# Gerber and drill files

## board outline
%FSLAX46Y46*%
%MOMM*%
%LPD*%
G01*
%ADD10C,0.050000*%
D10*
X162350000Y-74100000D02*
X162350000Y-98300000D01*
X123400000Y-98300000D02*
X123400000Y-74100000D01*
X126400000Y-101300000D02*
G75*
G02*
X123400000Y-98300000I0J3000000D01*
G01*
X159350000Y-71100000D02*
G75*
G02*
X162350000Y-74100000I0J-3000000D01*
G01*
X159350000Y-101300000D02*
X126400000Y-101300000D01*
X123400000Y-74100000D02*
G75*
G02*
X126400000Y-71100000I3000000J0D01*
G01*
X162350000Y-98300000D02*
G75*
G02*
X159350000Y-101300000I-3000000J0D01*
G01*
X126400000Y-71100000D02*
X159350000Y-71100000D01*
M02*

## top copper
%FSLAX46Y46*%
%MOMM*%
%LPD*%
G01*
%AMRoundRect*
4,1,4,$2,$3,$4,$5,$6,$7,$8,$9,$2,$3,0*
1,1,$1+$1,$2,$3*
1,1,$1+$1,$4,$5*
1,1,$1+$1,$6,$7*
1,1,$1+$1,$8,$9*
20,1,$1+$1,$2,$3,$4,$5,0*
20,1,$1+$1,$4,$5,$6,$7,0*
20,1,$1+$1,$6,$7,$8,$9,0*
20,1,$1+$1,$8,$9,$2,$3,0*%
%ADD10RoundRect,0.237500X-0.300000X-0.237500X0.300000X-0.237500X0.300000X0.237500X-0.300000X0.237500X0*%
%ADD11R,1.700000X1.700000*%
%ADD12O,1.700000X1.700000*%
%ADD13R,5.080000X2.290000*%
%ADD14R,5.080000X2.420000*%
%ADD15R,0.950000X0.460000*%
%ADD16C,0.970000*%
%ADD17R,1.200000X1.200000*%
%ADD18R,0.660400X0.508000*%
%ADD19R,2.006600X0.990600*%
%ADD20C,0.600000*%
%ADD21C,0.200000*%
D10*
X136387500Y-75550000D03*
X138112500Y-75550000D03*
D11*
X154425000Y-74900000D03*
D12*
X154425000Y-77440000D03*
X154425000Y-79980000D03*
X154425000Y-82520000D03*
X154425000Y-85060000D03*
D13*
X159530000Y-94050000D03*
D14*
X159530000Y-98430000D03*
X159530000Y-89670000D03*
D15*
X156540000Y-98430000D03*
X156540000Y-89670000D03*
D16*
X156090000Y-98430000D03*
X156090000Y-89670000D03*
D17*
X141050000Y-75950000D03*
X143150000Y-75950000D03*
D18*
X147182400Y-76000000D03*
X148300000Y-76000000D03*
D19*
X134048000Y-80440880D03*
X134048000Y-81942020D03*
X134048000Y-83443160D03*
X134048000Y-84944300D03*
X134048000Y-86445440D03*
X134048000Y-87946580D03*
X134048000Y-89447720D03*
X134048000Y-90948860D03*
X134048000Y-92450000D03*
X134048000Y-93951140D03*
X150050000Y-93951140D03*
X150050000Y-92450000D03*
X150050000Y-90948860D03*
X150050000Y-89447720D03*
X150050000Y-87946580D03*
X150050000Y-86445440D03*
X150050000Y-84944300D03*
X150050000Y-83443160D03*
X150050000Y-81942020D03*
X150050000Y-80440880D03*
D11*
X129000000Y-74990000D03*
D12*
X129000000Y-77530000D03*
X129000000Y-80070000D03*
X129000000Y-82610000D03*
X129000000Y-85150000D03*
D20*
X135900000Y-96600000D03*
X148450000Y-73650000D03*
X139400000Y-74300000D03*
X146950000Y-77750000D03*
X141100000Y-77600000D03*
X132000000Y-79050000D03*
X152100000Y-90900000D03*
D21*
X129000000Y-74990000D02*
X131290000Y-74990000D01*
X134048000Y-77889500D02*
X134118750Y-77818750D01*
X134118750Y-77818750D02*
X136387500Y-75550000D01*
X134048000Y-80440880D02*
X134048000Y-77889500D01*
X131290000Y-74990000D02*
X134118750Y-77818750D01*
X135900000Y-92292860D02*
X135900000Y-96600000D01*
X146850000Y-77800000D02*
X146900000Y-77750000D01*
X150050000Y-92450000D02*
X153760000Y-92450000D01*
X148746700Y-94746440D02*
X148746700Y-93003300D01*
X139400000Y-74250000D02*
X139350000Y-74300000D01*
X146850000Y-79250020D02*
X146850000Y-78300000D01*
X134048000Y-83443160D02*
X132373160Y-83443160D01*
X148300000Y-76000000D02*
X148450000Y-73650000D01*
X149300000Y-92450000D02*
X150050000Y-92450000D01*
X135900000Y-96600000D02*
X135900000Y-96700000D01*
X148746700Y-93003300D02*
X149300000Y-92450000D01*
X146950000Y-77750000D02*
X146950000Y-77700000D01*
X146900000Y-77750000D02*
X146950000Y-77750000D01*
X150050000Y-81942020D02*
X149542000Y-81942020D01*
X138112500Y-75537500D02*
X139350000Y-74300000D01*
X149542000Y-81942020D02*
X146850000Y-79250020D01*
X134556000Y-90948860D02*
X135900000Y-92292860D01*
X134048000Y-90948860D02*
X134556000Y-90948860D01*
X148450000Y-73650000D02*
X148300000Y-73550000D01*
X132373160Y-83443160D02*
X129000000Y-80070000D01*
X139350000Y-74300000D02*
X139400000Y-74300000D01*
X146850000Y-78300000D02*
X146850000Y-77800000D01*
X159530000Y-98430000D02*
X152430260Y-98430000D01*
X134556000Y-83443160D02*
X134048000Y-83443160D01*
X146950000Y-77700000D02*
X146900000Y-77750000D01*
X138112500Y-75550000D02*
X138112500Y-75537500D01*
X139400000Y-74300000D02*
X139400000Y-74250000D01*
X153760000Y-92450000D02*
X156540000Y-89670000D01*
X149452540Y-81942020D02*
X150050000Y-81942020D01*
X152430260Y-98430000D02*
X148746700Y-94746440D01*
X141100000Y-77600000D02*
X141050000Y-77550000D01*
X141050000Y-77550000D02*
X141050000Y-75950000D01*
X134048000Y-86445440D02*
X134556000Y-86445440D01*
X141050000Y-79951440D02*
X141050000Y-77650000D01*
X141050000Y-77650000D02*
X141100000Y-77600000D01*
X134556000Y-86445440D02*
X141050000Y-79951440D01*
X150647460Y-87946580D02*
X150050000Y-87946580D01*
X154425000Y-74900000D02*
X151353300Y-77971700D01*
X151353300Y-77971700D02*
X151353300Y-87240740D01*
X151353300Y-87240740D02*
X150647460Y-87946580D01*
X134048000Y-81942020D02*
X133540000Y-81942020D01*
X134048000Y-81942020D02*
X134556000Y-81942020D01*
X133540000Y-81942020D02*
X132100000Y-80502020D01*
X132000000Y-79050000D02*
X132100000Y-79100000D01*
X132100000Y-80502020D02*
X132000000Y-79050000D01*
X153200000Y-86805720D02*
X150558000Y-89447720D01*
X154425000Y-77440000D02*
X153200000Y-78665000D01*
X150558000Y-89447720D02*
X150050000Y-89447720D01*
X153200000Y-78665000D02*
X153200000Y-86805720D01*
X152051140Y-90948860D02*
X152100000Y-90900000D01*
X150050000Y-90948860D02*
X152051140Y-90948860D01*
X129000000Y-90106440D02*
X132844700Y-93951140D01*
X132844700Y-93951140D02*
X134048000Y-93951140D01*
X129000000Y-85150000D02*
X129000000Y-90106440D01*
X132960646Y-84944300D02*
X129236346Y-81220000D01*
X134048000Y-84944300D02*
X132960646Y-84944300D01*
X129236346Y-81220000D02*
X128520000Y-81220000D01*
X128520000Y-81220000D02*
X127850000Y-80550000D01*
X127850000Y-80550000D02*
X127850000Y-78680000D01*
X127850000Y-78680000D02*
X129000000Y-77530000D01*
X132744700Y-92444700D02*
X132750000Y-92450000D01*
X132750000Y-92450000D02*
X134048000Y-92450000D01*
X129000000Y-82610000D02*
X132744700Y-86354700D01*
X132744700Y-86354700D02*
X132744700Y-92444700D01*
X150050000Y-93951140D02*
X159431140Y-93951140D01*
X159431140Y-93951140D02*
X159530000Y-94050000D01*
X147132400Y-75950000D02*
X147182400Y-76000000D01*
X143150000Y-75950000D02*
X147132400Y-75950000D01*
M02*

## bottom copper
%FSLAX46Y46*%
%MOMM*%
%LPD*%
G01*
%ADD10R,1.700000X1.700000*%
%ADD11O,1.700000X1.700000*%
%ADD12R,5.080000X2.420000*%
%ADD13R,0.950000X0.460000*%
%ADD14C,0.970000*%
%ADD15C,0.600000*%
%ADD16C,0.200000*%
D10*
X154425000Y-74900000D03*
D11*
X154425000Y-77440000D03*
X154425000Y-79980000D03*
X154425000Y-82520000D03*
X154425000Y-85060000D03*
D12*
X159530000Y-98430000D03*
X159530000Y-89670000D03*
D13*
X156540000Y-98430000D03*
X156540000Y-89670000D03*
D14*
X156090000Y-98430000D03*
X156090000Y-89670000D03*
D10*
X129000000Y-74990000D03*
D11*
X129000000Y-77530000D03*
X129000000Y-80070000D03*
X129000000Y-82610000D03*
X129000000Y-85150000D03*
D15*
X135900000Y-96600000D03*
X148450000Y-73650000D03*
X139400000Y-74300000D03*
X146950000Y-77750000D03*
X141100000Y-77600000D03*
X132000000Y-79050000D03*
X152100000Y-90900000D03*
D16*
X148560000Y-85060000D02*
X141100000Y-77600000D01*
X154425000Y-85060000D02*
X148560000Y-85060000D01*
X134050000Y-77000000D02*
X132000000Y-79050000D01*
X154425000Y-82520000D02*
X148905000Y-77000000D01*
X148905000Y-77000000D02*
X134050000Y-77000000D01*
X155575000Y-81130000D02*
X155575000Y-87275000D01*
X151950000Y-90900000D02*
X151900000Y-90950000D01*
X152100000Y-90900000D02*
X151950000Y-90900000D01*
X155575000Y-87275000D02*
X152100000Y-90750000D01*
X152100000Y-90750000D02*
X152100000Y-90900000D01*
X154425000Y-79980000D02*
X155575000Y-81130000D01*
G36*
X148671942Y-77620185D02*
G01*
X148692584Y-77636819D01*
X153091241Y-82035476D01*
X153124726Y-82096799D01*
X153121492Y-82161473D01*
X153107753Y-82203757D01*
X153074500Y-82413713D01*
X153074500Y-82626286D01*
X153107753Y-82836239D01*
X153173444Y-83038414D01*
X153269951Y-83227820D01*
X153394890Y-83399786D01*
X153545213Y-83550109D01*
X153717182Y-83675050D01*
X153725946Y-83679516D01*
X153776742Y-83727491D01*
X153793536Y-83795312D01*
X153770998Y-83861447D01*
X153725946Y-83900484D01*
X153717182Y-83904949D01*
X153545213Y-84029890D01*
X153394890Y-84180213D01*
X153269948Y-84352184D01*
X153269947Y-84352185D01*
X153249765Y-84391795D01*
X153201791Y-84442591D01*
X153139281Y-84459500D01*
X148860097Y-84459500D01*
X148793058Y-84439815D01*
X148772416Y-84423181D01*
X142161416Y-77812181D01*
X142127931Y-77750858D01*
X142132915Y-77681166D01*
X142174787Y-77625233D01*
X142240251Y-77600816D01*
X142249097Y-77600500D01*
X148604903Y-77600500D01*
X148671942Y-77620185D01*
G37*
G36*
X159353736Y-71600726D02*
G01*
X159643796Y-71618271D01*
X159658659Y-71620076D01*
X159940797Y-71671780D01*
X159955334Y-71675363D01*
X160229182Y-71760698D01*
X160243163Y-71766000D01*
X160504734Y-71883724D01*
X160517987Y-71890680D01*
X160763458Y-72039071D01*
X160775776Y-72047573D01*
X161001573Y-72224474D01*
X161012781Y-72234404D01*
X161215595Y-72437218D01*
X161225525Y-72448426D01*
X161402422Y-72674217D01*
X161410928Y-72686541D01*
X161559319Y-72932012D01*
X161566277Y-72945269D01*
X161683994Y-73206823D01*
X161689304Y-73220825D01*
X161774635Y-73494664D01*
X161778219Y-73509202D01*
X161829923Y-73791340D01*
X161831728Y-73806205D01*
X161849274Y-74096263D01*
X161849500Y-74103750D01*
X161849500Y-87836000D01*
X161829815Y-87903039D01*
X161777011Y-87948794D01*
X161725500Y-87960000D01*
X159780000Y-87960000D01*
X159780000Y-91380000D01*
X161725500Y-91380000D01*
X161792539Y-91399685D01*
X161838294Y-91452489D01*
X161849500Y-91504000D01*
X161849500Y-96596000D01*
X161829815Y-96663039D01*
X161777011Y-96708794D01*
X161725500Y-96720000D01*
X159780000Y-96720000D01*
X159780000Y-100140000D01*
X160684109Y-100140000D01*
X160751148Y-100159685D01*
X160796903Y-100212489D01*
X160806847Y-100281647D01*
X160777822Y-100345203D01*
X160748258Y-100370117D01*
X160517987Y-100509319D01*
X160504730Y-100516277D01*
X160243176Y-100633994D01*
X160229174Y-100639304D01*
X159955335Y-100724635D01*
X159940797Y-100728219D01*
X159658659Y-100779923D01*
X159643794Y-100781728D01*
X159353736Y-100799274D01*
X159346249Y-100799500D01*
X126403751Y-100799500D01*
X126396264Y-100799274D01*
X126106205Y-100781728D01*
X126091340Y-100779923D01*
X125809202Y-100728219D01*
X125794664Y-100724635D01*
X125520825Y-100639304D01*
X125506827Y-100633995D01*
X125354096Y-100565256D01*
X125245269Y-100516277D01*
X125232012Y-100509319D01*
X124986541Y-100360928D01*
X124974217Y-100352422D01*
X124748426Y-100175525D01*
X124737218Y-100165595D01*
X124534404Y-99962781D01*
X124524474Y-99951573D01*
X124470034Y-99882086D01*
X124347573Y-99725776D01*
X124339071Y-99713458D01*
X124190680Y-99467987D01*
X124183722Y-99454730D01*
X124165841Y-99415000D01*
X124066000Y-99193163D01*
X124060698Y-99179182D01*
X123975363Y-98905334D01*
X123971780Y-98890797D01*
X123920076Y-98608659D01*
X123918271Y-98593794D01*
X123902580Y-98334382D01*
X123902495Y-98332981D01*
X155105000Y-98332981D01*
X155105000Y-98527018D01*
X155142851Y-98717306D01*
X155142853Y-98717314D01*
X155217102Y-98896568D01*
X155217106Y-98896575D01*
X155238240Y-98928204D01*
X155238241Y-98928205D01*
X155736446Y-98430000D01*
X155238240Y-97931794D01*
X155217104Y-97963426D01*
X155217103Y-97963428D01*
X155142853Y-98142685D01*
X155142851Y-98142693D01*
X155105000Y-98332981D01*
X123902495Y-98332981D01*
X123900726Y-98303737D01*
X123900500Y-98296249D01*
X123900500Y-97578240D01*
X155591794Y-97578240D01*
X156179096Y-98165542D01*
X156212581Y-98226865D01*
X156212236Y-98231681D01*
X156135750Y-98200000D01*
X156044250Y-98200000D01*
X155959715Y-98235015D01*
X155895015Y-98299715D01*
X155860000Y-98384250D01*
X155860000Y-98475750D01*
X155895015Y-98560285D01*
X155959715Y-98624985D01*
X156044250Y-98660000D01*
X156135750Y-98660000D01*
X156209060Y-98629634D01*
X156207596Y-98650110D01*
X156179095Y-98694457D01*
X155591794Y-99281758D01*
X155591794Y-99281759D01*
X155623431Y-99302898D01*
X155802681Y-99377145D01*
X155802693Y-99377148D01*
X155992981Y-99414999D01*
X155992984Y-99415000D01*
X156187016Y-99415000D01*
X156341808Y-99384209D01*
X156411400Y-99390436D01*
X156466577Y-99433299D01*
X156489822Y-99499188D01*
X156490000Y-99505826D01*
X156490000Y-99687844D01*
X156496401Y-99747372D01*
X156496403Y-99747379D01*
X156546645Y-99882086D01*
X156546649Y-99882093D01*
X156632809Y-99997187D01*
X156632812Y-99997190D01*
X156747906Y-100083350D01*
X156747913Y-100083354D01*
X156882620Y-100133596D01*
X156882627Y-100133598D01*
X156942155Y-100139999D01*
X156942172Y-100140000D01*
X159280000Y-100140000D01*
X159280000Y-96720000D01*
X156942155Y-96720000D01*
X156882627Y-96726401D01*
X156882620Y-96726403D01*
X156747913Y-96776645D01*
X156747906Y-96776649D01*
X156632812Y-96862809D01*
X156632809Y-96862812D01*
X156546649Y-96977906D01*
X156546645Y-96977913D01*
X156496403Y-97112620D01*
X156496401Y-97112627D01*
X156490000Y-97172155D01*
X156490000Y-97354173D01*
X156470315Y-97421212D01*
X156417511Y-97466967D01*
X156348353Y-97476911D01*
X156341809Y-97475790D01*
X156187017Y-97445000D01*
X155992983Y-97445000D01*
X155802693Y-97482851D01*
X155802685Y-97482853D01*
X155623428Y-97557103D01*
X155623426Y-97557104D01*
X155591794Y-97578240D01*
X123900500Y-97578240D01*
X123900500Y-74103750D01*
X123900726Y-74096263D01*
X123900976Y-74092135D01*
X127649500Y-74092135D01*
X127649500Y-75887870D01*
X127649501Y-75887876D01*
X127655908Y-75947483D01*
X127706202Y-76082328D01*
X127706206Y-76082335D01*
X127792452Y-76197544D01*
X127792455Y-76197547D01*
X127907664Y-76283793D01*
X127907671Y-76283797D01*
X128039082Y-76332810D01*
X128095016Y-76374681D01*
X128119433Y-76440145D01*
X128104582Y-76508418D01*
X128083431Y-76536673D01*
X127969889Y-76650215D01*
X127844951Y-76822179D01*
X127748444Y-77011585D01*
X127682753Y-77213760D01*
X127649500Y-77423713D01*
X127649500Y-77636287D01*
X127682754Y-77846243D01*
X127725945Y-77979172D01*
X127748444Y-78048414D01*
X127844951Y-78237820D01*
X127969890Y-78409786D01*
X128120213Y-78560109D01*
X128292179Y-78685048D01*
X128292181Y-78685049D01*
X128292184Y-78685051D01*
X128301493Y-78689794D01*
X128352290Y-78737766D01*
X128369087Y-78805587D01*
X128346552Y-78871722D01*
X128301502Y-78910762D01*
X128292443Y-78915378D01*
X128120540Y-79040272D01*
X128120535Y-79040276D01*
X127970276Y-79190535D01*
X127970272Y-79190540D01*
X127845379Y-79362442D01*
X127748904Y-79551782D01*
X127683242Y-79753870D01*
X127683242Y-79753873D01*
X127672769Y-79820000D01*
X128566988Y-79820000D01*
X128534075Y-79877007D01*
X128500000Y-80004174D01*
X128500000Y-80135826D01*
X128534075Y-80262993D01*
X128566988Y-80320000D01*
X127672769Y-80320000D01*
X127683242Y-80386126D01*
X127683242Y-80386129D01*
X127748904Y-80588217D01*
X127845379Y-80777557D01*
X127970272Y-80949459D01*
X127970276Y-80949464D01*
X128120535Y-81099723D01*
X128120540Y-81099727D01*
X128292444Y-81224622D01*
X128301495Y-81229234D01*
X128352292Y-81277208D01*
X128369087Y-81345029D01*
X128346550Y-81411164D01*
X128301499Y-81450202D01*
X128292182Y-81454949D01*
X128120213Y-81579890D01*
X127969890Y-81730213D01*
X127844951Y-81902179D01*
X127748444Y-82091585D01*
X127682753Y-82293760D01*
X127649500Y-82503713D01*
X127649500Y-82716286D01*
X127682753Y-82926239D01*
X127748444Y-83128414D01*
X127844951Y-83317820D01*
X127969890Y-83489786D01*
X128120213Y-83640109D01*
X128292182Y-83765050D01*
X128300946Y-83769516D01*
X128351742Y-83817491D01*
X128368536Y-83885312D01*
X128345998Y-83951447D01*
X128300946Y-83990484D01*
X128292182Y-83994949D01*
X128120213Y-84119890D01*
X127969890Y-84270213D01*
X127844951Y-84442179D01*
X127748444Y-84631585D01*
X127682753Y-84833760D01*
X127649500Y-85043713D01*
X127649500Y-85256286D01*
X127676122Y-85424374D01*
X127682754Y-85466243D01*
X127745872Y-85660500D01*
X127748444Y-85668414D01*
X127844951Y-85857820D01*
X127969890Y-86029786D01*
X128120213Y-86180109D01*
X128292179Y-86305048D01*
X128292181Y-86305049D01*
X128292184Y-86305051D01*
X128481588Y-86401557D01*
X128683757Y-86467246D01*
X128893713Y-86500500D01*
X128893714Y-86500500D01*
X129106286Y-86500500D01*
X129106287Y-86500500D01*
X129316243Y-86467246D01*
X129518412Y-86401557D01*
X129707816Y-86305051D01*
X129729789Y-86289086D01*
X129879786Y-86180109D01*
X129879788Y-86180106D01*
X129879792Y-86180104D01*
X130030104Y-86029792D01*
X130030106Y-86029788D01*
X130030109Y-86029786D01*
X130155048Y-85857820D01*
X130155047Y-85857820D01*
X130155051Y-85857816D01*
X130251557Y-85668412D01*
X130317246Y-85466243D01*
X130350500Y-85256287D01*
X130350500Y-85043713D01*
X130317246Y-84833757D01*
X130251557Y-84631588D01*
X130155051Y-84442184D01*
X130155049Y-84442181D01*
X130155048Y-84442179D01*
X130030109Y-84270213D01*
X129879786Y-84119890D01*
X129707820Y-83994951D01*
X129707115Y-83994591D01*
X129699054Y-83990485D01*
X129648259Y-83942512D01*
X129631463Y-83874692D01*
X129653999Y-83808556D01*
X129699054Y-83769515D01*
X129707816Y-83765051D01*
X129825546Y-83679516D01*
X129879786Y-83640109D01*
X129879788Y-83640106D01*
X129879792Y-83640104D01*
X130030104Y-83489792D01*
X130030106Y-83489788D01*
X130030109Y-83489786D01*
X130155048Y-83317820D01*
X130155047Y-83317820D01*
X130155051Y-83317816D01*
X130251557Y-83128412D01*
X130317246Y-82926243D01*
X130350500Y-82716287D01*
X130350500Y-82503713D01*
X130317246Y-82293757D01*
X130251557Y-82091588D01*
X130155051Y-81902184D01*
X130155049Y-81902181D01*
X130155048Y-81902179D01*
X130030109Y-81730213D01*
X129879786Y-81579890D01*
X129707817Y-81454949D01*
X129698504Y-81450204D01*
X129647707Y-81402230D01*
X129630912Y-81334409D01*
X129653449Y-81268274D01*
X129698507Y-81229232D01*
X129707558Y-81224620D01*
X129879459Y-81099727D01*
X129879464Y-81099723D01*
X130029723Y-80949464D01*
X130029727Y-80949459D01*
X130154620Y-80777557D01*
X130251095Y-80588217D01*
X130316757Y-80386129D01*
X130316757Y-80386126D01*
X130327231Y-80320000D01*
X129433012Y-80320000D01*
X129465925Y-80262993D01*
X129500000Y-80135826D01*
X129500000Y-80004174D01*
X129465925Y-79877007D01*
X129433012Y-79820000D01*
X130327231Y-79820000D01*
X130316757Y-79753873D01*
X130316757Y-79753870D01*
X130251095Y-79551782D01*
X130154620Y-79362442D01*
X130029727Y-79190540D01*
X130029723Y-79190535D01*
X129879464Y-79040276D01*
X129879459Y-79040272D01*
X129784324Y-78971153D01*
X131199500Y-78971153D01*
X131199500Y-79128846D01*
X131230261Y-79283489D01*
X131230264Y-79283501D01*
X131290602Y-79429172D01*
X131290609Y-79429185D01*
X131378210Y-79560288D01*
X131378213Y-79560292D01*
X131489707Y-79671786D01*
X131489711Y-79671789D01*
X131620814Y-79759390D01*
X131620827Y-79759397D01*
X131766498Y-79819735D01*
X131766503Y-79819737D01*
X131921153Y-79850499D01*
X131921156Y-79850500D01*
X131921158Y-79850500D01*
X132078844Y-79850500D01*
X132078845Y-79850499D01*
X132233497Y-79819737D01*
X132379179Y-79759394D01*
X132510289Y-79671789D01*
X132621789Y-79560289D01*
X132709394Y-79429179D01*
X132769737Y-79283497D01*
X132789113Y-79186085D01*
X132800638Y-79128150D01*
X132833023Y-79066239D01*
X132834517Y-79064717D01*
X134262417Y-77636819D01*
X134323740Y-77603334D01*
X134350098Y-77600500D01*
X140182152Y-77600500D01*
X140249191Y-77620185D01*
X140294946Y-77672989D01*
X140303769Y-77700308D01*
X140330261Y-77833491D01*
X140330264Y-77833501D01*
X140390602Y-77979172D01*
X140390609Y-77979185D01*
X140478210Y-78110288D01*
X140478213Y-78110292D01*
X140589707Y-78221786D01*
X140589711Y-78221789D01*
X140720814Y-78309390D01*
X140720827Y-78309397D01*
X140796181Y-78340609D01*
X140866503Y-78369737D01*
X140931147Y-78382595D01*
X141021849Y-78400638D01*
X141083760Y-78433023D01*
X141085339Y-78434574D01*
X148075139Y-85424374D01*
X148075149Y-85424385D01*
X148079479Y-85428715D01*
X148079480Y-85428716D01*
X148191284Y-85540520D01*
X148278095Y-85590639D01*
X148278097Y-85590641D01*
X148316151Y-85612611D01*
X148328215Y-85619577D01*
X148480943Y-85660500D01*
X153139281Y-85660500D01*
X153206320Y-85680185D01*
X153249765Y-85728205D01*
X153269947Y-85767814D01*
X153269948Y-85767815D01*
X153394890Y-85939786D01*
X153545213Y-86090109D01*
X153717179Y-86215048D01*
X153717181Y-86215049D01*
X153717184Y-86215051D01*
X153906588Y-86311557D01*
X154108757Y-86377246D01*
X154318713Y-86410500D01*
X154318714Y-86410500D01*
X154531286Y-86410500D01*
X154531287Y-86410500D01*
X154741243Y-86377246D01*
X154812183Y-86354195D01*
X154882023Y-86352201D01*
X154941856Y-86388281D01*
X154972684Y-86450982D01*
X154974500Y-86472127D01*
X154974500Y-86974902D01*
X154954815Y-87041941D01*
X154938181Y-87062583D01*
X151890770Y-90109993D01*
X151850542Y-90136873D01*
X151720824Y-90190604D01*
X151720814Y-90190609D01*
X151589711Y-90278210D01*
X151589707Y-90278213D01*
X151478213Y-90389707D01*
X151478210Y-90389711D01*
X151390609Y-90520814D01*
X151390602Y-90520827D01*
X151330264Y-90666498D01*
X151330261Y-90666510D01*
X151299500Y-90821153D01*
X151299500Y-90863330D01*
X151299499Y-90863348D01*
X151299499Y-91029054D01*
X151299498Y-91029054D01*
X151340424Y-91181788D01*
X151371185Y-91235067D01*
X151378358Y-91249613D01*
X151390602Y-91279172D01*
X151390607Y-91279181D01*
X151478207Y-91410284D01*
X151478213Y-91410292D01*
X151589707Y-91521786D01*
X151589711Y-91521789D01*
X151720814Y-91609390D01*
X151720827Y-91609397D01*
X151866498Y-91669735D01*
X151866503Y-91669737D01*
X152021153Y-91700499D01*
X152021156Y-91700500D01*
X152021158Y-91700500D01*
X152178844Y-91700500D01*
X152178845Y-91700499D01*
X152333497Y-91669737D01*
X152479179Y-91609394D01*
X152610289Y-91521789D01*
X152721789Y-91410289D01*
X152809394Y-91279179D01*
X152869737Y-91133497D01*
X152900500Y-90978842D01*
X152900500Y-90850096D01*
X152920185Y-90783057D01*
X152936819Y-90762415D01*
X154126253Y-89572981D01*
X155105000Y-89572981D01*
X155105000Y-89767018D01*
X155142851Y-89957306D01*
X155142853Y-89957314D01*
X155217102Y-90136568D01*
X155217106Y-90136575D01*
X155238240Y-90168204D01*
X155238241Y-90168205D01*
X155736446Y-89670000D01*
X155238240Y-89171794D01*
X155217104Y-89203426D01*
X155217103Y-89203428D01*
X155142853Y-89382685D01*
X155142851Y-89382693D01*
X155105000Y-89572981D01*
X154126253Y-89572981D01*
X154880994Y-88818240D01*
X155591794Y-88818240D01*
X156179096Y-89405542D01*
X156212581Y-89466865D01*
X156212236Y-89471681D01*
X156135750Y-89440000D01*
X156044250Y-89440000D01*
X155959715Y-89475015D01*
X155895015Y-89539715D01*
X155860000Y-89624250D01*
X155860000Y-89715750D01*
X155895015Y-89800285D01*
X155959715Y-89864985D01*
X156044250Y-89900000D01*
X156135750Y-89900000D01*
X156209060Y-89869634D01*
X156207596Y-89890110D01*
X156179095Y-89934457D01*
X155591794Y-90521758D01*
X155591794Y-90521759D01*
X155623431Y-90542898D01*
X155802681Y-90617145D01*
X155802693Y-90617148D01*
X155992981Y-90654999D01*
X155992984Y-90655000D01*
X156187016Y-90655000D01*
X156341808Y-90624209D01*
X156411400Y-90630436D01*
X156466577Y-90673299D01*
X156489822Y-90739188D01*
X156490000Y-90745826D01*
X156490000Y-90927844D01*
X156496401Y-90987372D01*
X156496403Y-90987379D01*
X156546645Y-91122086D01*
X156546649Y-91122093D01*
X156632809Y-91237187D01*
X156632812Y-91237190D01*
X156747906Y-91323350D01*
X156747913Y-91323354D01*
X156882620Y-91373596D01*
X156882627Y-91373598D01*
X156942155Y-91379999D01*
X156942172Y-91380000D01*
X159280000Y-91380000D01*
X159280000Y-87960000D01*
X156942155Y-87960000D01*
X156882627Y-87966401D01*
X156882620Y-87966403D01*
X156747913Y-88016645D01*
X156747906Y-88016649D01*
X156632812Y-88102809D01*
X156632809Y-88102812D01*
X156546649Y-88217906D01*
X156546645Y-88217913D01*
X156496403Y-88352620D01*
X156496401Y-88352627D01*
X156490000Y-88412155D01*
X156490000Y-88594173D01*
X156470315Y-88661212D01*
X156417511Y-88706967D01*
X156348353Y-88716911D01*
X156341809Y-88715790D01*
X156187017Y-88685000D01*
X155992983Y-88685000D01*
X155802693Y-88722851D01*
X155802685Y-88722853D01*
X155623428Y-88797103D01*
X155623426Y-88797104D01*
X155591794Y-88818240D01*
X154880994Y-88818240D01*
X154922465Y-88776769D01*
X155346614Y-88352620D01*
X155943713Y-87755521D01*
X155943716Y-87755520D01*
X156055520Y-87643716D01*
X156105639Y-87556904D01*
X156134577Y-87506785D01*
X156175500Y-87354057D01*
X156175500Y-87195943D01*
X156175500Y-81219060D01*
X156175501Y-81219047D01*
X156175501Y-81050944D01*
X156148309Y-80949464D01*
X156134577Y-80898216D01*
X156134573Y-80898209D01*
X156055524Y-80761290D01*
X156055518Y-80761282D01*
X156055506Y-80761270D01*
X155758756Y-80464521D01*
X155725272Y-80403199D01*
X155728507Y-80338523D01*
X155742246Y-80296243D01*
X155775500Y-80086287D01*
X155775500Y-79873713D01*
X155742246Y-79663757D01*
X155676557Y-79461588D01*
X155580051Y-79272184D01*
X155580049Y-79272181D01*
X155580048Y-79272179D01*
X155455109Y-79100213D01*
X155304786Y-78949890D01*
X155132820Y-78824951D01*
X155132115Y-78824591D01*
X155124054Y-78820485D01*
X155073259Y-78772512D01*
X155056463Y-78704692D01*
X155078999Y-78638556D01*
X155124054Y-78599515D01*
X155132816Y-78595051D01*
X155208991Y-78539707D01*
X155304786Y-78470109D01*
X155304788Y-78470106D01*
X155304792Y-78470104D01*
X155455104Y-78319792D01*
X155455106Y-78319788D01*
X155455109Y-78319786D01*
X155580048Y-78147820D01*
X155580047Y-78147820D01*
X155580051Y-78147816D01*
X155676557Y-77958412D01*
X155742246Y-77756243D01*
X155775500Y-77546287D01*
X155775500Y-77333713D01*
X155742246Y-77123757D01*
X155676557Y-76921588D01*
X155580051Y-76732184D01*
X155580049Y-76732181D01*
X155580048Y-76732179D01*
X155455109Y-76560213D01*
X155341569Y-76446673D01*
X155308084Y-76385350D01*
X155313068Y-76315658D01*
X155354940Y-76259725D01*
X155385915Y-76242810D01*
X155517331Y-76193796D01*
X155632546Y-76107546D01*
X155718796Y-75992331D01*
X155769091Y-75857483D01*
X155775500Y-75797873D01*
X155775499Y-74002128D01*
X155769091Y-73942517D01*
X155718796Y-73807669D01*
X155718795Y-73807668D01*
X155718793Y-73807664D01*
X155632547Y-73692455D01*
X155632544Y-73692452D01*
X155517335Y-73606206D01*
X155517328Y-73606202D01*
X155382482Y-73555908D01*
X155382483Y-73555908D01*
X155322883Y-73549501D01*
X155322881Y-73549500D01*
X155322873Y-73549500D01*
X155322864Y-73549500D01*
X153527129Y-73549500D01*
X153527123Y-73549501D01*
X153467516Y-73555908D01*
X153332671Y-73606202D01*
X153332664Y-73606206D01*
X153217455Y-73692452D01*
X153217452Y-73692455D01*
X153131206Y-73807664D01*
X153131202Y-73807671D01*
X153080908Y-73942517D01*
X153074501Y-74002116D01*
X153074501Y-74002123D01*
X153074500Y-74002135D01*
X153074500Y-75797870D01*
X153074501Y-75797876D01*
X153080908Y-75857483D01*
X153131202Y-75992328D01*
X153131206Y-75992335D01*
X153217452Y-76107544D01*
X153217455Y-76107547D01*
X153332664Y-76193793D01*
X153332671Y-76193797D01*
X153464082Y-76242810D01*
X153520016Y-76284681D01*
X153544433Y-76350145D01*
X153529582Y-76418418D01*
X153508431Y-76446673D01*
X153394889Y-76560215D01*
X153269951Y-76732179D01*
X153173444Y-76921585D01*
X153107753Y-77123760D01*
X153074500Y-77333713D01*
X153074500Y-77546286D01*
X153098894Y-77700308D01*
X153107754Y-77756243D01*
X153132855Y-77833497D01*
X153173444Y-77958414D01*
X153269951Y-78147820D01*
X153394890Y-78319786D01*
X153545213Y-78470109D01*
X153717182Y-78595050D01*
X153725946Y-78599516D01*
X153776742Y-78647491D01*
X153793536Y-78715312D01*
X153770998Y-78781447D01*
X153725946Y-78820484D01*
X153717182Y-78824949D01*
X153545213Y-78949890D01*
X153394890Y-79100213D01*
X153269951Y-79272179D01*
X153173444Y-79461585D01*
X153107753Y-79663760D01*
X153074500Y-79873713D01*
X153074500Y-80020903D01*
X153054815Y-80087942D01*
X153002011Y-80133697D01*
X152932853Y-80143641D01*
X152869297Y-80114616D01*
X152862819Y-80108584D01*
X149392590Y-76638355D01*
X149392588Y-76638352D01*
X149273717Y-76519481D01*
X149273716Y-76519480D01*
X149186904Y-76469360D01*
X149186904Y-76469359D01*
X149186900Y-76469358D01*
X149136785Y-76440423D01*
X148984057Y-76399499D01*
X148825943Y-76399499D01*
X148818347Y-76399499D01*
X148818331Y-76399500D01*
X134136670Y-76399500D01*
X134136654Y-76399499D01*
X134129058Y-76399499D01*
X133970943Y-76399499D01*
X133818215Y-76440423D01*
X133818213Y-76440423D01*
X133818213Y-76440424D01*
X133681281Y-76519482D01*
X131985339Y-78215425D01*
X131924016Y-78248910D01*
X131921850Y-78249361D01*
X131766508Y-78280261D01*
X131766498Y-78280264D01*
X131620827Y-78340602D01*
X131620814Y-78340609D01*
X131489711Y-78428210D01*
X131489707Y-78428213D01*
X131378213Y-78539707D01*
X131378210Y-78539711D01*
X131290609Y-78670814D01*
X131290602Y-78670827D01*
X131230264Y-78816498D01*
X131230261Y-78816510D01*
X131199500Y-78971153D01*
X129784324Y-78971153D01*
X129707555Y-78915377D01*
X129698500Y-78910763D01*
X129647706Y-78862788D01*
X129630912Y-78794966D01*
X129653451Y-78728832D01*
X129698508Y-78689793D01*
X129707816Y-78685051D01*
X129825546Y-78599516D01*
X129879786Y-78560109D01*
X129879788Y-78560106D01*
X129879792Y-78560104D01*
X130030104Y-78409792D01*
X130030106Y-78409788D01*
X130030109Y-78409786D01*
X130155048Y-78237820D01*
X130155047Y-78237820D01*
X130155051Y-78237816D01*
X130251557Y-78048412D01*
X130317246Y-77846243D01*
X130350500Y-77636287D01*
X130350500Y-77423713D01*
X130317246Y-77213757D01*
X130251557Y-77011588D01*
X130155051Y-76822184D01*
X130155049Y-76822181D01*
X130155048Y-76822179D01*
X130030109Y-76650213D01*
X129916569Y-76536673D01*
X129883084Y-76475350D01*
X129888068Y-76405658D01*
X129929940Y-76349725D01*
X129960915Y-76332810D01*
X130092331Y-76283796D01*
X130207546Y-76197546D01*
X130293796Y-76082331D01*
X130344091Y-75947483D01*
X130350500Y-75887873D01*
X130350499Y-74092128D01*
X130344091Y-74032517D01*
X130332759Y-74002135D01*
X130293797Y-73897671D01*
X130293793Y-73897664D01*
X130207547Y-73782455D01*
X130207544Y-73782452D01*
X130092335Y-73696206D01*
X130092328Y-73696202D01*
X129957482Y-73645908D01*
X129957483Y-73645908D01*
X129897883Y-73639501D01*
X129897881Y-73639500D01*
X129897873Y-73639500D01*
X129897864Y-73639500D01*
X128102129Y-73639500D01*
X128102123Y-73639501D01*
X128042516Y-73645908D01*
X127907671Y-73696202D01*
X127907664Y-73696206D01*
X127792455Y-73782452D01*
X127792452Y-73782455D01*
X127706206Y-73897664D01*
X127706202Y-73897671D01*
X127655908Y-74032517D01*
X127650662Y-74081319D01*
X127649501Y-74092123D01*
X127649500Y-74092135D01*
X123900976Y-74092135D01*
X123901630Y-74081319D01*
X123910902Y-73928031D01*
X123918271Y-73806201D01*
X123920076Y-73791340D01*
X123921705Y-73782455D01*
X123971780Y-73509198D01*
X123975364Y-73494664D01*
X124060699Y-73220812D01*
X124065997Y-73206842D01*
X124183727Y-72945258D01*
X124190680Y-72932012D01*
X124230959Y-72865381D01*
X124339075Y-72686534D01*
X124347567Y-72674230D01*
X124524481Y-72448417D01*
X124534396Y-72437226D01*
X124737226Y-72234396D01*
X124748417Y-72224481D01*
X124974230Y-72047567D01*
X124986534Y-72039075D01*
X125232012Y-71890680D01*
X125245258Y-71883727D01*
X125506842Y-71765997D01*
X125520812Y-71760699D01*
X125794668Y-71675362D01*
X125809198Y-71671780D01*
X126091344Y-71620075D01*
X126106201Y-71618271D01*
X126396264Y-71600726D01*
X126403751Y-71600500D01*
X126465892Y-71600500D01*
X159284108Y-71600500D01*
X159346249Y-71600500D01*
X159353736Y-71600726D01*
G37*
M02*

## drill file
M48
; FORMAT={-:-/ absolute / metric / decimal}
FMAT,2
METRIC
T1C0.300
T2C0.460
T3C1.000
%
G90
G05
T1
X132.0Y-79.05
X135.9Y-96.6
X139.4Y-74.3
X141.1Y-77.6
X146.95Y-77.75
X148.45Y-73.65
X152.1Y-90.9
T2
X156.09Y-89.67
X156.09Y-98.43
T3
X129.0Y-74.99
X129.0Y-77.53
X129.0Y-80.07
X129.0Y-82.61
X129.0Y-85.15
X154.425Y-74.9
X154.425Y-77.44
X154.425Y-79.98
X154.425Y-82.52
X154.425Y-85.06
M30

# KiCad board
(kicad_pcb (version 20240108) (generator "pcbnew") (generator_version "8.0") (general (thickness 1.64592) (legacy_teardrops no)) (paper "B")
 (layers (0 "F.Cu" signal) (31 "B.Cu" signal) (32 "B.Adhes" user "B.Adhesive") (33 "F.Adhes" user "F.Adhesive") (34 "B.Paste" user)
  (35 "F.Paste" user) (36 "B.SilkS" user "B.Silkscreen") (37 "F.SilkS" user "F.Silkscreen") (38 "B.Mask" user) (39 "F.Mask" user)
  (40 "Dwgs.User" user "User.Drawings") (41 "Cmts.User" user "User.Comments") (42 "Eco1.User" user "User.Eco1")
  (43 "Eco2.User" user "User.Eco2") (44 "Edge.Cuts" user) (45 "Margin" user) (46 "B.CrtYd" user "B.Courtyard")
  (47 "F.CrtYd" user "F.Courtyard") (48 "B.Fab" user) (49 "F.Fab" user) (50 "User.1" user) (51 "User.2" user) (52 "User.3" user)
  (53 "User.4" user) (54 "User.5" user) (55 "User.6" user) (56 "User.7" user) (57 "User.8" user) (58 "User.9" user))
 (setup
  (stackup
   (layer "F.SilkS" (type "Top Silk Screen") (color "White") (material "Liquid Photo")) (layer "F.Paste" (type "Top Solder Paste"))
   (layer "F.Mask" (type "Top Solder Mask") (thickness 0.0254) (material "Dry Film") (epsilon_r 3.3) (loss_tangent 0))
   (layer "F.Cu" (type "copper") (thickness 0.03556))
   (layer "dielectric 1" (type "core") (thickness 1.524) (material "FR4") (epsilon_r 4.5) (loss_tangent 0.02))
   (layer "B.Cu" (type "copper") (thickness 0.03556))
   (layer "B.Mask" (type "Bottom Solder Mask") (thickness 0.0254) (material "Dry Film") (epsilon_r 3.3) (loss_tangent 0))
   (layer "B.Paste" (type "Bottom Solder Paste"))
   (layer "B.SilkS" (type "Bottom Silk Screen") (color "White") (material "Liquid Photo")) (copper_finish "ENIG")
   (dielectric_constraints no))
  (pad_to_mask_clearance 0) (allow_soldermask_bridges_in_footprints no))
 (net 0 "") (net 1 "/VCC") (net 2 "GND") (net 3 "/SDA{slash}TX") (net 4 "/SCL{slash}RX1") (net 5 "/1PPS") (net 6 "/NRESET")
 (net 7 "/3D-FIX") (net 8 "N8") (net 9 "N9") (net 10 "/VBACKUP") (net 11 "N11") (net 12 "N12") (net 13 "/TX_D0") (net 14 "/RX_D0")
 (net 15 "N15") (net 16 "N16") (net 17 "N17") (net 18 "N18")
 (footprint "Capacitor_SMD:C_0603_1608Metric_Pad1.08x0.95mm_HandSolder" (layer "F.Cu") (at 137.25 75.55)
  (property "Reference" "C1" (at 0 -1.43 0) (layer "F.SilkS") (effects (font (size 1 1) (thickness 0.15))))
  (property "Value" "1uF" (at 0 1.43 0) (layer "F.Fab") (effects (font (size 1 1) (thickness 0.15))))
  (pad "1" smd roundrect (at -0.8625 0) (size 1.075 0.95) (layers "F.Cu" "F.Paste" "F.Mask") (roundrect_rratio 0.25) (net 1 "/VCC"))
  (pad "2" smd roundrect (at 0.8625 0) (size 1.075 0.95) (layers "F.Cu" "F.Paste" "F.Mask") (roundrect_rratio 0.25) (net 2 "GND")))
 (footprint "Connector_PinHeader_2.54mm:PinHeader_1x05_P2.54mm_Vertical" (layer "F.Cu") (at 154.425 74.9)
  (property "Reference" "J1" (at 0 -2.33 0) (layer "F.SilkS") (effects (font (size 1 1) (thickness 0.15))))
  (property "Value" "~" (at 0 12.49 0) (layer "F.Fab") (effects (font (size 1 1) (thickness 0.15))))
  (pad "1" thru_hole rect (at 0 0) (size 1.7 1.7) (drill 1) (layers "*.Cu" "*.Mask") (remove_unused_layers no) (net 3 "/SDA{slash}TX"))
  (pad "2" thru_hole oval (at 0 2.54) (size 1.7 1.7) (drill 1) (layers "*.Cu" "*.Mask") (remove_unused_layers no) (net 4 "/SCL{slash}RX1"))
  (pad "3" thru_hole oval (at 0 5.08) (size 1.7 1.7) (drill 1) (layers "*.Cu" "*.Mask") (remove_unused_layers no) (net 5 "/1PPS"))
  (pad "4" thru_hole oval (at 0 7.62) (size 1.7 1.7) (drill 1) (layers "*.Cu" "*.Mask") (remove_unused_layers no) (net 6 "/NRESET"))
  (pad "5" thru_hole oval (at 0 10.16) (size 1.7 1.7) (drill 1) (layers "*.Cu" "*.Mask") (remove_unused_layers no) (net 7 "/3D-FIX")))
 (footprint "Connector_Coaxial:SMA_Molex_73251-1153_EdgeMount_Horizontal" (layer "F.Cu") (at 157.81 94.05 180)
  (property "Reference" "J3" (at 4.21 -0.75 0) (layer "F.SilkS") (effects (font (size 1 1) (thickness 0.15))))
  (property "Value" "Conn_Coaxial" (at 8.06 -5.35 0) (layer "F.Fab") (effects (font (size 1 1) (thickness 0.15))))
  (pad "1" smd rect (at -1.72 0 180) (size 5.08 2.29) (layers "F.Cu" "F.Paste" "F.Mask") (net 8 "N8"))
  (pad "2" smd rect (at -1.72 -4.38 180) (size 5.08 2.42) (layers "F.Cu" "F.Paste" "F.Mask") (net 2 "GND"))
  (pad "2" smd rect (at -1.72 -4.38 180) (size 5.08 2.42) (layers "B.Cu" "B.Paste" "B.Mask") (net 2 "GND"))
  (pad "2" smd rect (at -1.72 4.38 180) (size 5.08 2.42) (layers "F.Cu" "F.Paste" "F.Mask") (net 2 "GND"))
  (pad "2" smd rect (at -1.72 4.38 180) (size 5.08 2.42) (layers "B.Cu" "B.Paste" "B.Mask") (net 2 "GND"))
  (pad "2" smd rect (at 1.27 -4.38 180) (size 0.95 0.46) (layers "F.Cu") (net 2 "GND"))
  (pad "2" smd rect (at 1.27 -4.38 180) (size 0.95 0.46) (layers "B.Cu") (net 2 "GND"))
  (pad "2" smd rect (at 1.27 4.38 180) (size 0.95 0.46) (layers "F.Cu") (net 2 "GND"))
  (pad "2" smd rect (at 1.27 4.38 180) (size 0.95 0.46) (layers "B.Cu") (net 2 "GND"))
  (pad "2" thru_hole circle (at 1.72 -4.38 180) (size 0.97 0.97) (drill 0.46) (layers "*.Cu") (remove_unused_layers no) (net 2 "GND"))
  (pad "2" thru_hole circle (at 1.72 4.38 180) (size 0.97 0.97) (drill 0.46) (layers "*.Cu") (remove_unused_layers no) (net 2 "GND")))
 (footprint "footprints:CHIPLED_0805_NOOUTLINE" (layer "F.Cu") (at 142.1 75.95 -90)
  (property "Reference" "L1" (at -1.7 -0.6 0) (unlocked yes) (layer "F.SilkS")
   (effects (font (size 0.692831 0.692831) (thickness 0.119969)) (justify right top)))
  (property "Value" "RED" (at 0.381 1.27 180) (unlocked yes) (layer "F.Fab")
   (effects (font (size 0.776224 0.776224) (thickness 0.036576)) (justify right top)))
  (pad "A" smd rect (at 0 1.05 270) (size 1.2 1.2) (layers "F.Cu" "F.Paste" "F.Mask") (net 7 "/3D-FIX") (solder_mask_margin 0.0508)
   (thermal_bridge_angle 0))
  (pad "C" smd rect (at 0 -1.05 270) (size 1.2 1.2) (layers "F.Cu" "F.Paste" "F.Mask") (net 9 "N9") (solder_mask_margin 0.0508)
   (thermal_bridge_angle 0)))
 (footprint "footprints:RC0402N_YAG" (layer "F.Cu") (at 147.7412 76)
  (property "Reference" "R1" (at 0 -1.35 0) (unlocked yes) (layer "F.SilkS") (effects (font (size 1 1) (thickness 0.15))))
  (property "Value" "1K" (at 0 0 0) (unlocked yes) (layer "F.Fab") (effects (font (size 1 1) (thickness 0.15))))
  (pad "1" smd rect (at -0.5588 0) (size 0.6604 0.508) (layers "F.Cu" "F.Paste" "F.Mask") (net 9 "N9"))
  (pad "2" smd rect (at 0.5588 0) (size 0.6604 0.508) (layers "F.Cu" "F.Paste" "F.Mask") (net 2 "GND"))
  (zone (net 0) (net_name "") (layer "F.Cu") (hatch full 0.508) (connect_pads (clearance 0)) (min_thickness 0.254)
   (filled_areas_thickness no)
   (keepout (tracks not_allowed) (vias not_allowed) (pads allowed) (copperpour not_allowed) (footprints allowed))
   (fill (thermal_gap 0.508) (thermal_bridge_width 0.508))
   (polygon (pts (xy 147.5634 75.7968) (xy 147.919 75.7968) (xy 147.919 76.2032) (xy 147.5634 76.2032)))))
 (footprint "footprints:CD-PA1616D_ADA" (layer "F.Cu") (at 142.049 87.19601)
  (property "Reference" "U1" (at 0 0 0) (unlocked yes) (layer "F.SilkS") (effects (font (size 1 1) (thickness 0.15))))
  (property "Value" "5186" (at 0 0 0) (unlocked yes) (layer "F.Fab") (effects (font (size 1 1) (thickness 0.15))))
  (pad "1" smd rect (at -8.001 -6.75513) (size 2.0066 0.9906) (layers "F.Cu" "F.Paste" "F.Mask") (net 1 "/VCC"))
  (pad "2" smd rect (at -8.001 -5.25399) (size 2.0066 0.9906) (layers "F.Cu" "F.Paste" "F.Mask") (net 6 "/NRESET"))
  (pad "3" smd rect (at -8.001 -3.75285) (size 2.0066 0.9906) (layers "F.Cu" "F.Paste" "F.Mask") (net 2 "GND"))
  (pad "4" smd rect (at -8.001 -2.25171) (size 2.0066 0.9906) (layers "F.Cu" "F.Paste" "F.Mask") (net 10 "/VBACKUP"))
  (pad "5" smd rect (at -8.001 -0.75057) (size 2.0066 0.9906) (layers "F.Cu" "F.Paste" "F.Mask") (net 7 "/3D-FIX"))
  (pad "6" smd rect (at -8.001 0.75057) (size 2.0066 0.9906) (layers "F.Cu" "F.Paste" "F.Mask") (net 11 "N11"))
  (pad "7" smd rect (at -8.001 2.25171) (size 2.0066 0.9906) (layers "F.Cu" "F.Paste" "F.Mask") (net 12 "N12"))
  (pad "8" smd rect (at -8.001 3.75285) (size 2.0066 0.9906) (layers "F.Cu" "F.Paste" "F.Mask") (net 2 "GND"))
  (pad "9" smd rect (at -8.001 5.25399) (size 2.0066 0.9906) (layers "F.Cu" "F.Paste" "F.Mask") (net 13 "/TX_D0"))
  (pad "10" smd rect (at -8.001 6.75513) (size 2.0066 0.9906) (layers "F.Cu" "F.Paste" "F.Mask") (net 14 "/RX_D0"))
  (pad "11" smd rect (at 8.001 6.75513) (size 2.0066 0.9906) (layers "F.Cu" "F.Paste" "F.Mask") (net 8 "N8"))
  (pad "12" smd rect (at 8.001 5.25399) (size 2.0066 0.9906) (layers "F.Cu" "F.Paste" "F.Mask") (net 2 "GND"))
  (pad "13" smd rect (at 8.001 3.75285) (size 2.0066 0.9906) (layers "F.Cu" "F.Paste" "F.Mask") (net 5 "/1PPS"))
  (pad "14" smd rect (at 8.001 2.25171) (size 2.0066 0.9906) (layers "F.Cu" "F.Paste" "F.Mask") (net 4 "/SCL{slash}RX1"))
  (pad "15" smd rect (at 8.001 0.75057) (size 2.0066 0.9906) (layers "F.Cu" "F.Paste" "F.Mask") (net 3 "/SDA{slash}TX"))
  (pad "16" smd rect (at 8.001 -0.75057) (size 2.0066 0.9906) (layers "F.Cu" "F.Paste" "F.Mask") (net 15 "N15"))
  (pad "17" smd rect (at 8.001 -2.25171) (size 2.0066 0.9906) (layers "F.Cu" "F.Paste" "F.Mask") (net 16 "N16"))
  (pad "18" smd rect (at 8.001 -3.75285) (size 2.0066 0.9906) (layers "F.Cu" "F.Paste" "F.Mask") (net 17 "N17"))
  (pad "19" smd rect (at 8.001 -5.25399) (size 2.0066 0.9906) (layers "F.Cu" "F.Paste" "F.Mask") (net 2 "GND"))
  (pad "20" smd rect (at 8.001 -6.75513) (size 2.0066 0.9906) (layers "F.Cu" "F.Paste" "F.Mask") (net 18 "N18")))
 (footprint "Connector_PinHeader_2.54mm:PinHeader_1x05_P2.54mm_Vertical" (layer "F.Cu") (at 129 74.99)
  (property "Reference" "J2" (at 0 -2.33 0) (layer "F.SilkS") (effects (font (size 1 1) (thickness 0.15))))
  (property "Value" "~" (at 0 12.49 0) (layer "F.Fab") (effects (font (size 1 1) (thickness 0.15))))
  (pad "1" thru_hole rect (at 0 0) (size 1.7 1.7) (drill 1) (layers "*.Cu" "*.Mask") (remove_unused_layers no) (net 1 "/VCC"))
  (pad "2" thru_hole oval (at 0 2.54) (size 1.7 1.7) (drill 1) (layers "*.Cu" "*.Mask") (remove_unused_layers no) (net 10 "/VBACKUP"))
  (pad "3" thru_hole oval (at 0 5.08) (size 1.7 1.7) (drill 1) (layers "*.Cu" "*.Mask") (remove_unused_layers no) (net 2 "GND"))
  (pad "4" thru_hole oval (at 0 7.62) (size 1.7 1.7) (drill 1) (layers "*.Cu" "*.Mask") (remove_unused_layers no) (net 13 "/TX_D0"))
  (pad "5" thru_hole oval (at 0 10.16) (size 1.7 1.7) (drill 1) (layers "*.Cu" "*.Mask") (remove_unused_layers no) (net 14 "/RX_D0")))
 (gr_line (start 162.35 74.1) (end 162.35 98.3) (stroke (width 0.05) (type default)) (layer "Edge.Cuts"))
 (gr_line (start 123.4 98.3) (end 123.4 74.1) (stroke (width 0.05) (type default)) (layer "Edge.Cuts"))
 (gr_arc (start 126.4 101.3) (mid 124.27868 100.42132) (end 123.4 98.3) (stroke (width 0.05) (type default)) (layer "Edge.Cuts"))
 (gr_arc (start 159.35 71.1) (mid 161.47132 71.97868) (end 162.35 74.1) (stroke (width 0.05) (type default)) (layer "Edge.Cuts"))
 (gr_line (start 159.35 101.3) (end 126.4 101.3) (stroke (width 0.05) (type default)) (layer "Edge.Cuts"))
 (gr_arc (start 123.4 74.1) (mid 124.27868 71.97868) (end 126.4 71.1) (stroke (width 0.05) (type default)) (layer "Edge.Cuts"))
 (gr_arc (start 162.35 98.3) (mid 161.47132 100.42132) (end 159.35 101.3) (stroke (width 0.05) (type default)) (layer "Edge.Cuts"))
 (gr_line (start 126.4 71.1) (end 159.35 71.1) (stroke (width 0.05) (type default)) (layer "Edge.Cuts"))
 (segment (start 129 74.99) (end 131.29 74.99) (width 0.2) (layer "F.Cu") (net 1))
 (segment (start 134.048 77.8895) (end 134.11875 77.81875) (width 0.2) (layer "F.Cu") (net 1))
 (segment (start 134.11875 77.81875) (end 136.3875 75.55) (width 0.2) (layer "F.Cu") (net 1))
 (segment (start 134.048 80.44088) (end 134.048 77.8895) (width 0.2) (layer "F.Cu") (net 1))
 (segment (start 131.29 74.99) (end 134.11875 77.81875) (width 0.2) (layer "F.Cu") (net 1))
 (segment (start 135.9 92.29286) (end 135.9 96.6) (width 0.2) (layer "F.Cu") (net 2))
 (segment (start 146.85 77.8) (end 146.9 77.75) (width 0.2) (layer "F.Cu") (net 2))
 (segment (start 150.05 92.45) (end 153.76 92.45) (width 0.2) (layer "F.Cu") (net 2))
 (segment (start 148.7467 94.74644) (end 148.7467 93.0033) (width 0.2) (layer "F.Cu") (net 2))
 (segment (start 139.4 74.25) (end 139.35 74.3) (width 0.2) (layer "F.Cu") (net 2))
 (segment (start 146.85 79.25002) (end 146.85 78.3) (width 0.2) (layer "F.Cu") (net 2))
 (segment (start 134.048 83.44316) (end 132.37316 83.44316) (width 0.2) (layer "F.Cu") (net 2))
 (segment (start 148.3 76) (end 148.45 73.65) (width 0.2) (layer "F.Cu") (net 2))
 (segment (start 149.3 92.45) (end 150.05 92.45) (width 0.2) (layer "F.Cu") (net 2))
 (segment (start 135.9 96.6) (end 135.9 96.7) (width 0.2) (layer "F.Cu") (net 2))
 (segment (start 148.7467 93.0033) (end 149.3 92.45) (width 0.2) (layer "F.Cu") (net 2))
 (segment (start 146.95 77.75) (end 146.95 77.7) (width 0.2) (layer "F.Cu") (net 2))
 (segment (start 146.9 77.75) (end 146.95 77.75) (width 0.2) (layer "F.Cu") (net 2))
 (segment (start 150.05 81.94202) (end 149.542 81.94202) (width 0.2) (layer "F.Cu") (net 2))
 (segment (start 138.1125 75.5375) (end 139.35 74.3) (width 0.2) (layer "F.Cu") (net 2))
 (segment (start 149.542 81.94202) (end 146.85 79.25002) (width 0.2) (layer "F.Cu") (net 2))
 (segment (start 134.556 90.94886) (end 135.9 92.29286) (width 0.2) (layer "F.Cu") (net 2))
 (segment (start 134.048 90.94886) (end 134.556 90.94886) (width 0.2) (layer "F.Cu") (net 2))
 (segment (start 148.45 73.65) (end 148.3 73.55) (width 0.2) (layer "F.Cu") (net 2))
 (segment (start 132.37316 83.44316) (end 129 80.07) (width 0.2) (layer "F.Cu") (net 2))
 (segment (start 139.35 74.3) (end 139.4 74.3) (width 0.2) (layer "F.Cu") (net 2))
 (segment (start 146.85 78.3) (end 146.85 77.8) (width 0.2) (layer "F.Cu") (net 2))
 (segment (start 159.53 98.43) (end 152.43026 98.43) (width 0.2) (layer "F.Cu") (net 2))
 (segment (start 134.556 83.44316) (end 134.048 83.44316) (width 0.2) (layer "F.Cu") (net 2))
 (segment (start 146.95 77.7) (end 146.9 77.75) (width 0.2) (layer "F.Cu") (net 2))
 (segment (start 138.1125 75.55) (end 138.1125 75.5375) (width 0.2) (layer "F.Cu") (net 2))
 (segment (start 139.4 74.3) (end 139.4 74.25) (width 0.2) (layer "F.Cu") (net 2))
 (segment (start 153.76 92.45) (end 156.54 89.67) (width 0.2) (layer "F.Cu") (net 2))
 (segment (start 149.45254 81.94202) (end 150.05 81.94202) (width 0.2) (layer "F.Cu") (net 2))
 (segment (start 152.43026 98.43) (end 148.7467 94.74644) (width 0.2) (layer "F.Cu") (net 2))
 (via (at 135.9 96.6) (size 0.6) (drill 0.3) (layers "F.Cu" "B.Cu") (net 2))
 (via (at 148.45 73.65) (size 0.6) (drill 0.3) (layers "F.Cu" "B.Cu") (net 2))
 (via (at 139.4 74.3) (size 0.6) (drill 0.3) (layers "F.Cu" "B.Cu") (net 2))
 (via (at 146.95 77.75) (size 0.6) (drill 0.3) (layers "F.Cu" "B.Cu") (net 2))
 (segment (start 141.1 77.6) (end 141.05 77.55) (width 0.2) (layer "F.Cu") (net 7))
 (segment (start 141.05 77.55) (end 141.05 75.95) (width 0.2) (layer "F.Cu") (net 7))
 (segment (start 134.048 86.44544) (end 134.556 86.44544) (width 0.2) (layer "F.Cu") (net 7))
 (segment (start 141.05 79.95144) (end 141.05 77.65) (width 0.2) (layer "F.Cu") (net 7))
 (segment (start 141.05 77.65) (end 141.1 77.6) (width 0.2) (layer "F.Cu") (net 7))
 (segment (start 134.556 86.44544) (end 141.05 79.95144) (width 0.2) (layer "F.Cu") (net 7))
 (via (at 141.1 77.6) (size 0.6) (drill 0.3) (layers "F.Cu" "B.Cu") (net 7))
 (segment (start 148.56 85.06) (end 141.1 77.6) (width 0.2) (layer "B.Cu") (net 7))
 (segment (start 154.425 85.06) (end 148.56 85.06) (width 0.2) (layer "B.Cu") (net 7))
 (segment (start 150.64746 87.94658) (end 150.05 87.94658) (width 0.2) (layer "F.Cu") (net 3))
 (segment (start 154.425 74.9) (end 151.3533 77.9717) (width 0.2) (layer "F.Cu") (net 3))
 (segment (start 151.3533 77.9717) (end 151.3533 87.24074) (width 0.2) (layer "F.Cu") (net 3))
 (segment (start 151.3533 87.24074) (end 150.64746 87.94658) (width 0.2) (layer "F.Cu") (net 3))
 (segment (start 134.048 81.94202) (end 133.54 81.94202) (width 0.2) (layer "F.Cu") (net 6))
 (segment (start 134.048 81.94202) (end 134.556 81.94202) (width 0.2) (layer "F.Cu") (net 6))
 (segment (start 133.54 81.94202) (end 132.1 80.50202) (width 0.2) (layer "F.Cu") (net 6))
 (segment (start 132 79.05) (end 132.1 79.1) (width 0.2) (layer "F.Cu") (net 6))
 (segment (start 132.1 80.50202) (end 132 79.05) (width 0.2) (layer "F.Cu") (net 6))
 (via (at 132 79.05) (size 0.6) (drill 0.3) (layers "F.Cu" "B.Cu") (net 6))
 (segment (start 134.05 77) (end 132 79.05) (width 0.2) (layer "B.Cu") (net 6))
 (segment (start 154.425 82.52) (end 148.905 77) (width 0.2) (layer "B.Cu") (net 6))
 (segment (start 148.905 77) (end 134.05 77) (width 0.2) (layer "B.Cu") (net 6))
 (segment (start 153.2 86.80572) (end 150.558 89.44772) (width 0.2) (layer "F.Cu") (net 4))
 (segment (start 154.425 77.44) (end 153.2 78.665) (width 0.2) (layer "F.Cu") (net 4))
 (segment (start 150.558 89.44772) (end 150.05 89.44772) (width 0.2) (layer "F.Cu") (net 4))
 (segment (start 153.2 78.665) (end 153.2 86.80572) (width 0.2) (layer "F.Cu") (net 4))
 (segment (start 152.05114 90.94886) (end 152.1 90.9) (width 0.2) (layer "F.Cu") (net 5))
 (segment (start 150.05 90.94886) (end 152.05114 90.94886) (width 0.2) (layer "F.Cu") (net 5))
 (via (at 152.1 90.9) (size 0.6) (drill 0.3) (layers "F.Cu" "B.Cu") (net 5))
 (segment (start 155.575 81.13) (end 155.575 87.275) (width 0.2) (layer "B.Cu") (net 5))
 (segment (start 151.95 90.9) (end 151.9 90.95) (width 0.2) (layer "B.Cu") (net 5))
 (segment (start 152.1 90.9) (end 151.95 90.9) (width 0.2) (layer "B.Cu") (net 5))
 (segment (start 155.575 87.275) (end 152.1 90.75) (width 0.2) (layer "B.Cu") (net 5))
 (segment (start 152.1 90.75) (end 152.1 90.9) (width 0.2) (layer "B.Cu") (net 5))
 (segment (start 154.425 79.98) (end 155.575 81.13) (width 0.2) (layer "B.Cu") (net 5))
 (segment (start 129 90.10644) (end 132.8447 93.95114) (width 0.2) (layer "F.Cu") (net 14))
 (segment (start 132.8447 93.95114) (end 134.048 93.95114) (width 0.2) (layer "F.Cu") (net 14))
 (segment (start 129 85.15) (end 129 90.10644) (width 0.2) (layer "F.Cu") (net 14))
 (segment (start 132.960646 84.9443) (end 129.236346 81.22) (width 0.2) (layer "F.Cu") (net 10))
 (segment (start 134.048 84.9443) (end 132.960646 84.9443) (width 0.2) (layer "F.Cu") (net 10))
 (segment (start 129.236346 81.22) (end 128.52 81.22) (width 0.2) (layer "F.Cu") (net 10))
 (segment (start 128.52 81.22) (end 127.85 80.55) (width 0.2) (layer "F.Cu") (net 10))
 (segment (start 127.85 80.55) (end 127.85 78.68) (width 0.2) (layer "F.Cu") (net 10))
 (segment (start 127.85 78.68) (end 129 77.53) (width 0.2) (layer "F.Cu") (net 10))
 (segment (start 132.7447 92.4447) (end 132.75 92.45) (width 0.2) (layer "F.Cu") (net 13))
 (segment (start 132.75 92.45) (end 134.048 92.45) (width 0.2) (layer "F.Cu") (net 13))
 (segment (start 129 82.61) (end 132.7447 86.3547) (width 0.2) (layer "F.Cu") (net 13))
 (segment (start 132.7447 86.3547) (end 132.7447 92.4447) (width 0.2) (layer "F.Cu") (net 13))
 (segment (start 150.05 93.95114) (end 159.43114 93.95114) (width 0.2) (layer "F.Cu") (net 8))
 (segment (start 159.43114 93.95114) (end 159.53 94.05) (width 0.2) (layer "F.Cu") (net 8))
 (segment (start 147.1324 75.95) (end 147.1824 76) (width 0.2) (layer "F.Cu") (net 9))
 (segment (start 143.15 75.95) (end 147.1324 75.95) (width 0.2) (layer "F.Cu") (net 9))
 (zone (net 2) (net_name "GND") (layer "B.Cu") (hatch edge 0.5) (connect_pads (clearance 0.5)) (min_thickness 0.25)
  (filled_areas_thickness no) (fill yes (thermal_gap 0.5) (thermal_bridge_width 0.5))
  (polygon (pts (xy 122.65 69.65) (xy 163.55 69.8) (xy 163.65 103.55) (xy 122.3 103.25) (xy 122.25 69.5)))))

